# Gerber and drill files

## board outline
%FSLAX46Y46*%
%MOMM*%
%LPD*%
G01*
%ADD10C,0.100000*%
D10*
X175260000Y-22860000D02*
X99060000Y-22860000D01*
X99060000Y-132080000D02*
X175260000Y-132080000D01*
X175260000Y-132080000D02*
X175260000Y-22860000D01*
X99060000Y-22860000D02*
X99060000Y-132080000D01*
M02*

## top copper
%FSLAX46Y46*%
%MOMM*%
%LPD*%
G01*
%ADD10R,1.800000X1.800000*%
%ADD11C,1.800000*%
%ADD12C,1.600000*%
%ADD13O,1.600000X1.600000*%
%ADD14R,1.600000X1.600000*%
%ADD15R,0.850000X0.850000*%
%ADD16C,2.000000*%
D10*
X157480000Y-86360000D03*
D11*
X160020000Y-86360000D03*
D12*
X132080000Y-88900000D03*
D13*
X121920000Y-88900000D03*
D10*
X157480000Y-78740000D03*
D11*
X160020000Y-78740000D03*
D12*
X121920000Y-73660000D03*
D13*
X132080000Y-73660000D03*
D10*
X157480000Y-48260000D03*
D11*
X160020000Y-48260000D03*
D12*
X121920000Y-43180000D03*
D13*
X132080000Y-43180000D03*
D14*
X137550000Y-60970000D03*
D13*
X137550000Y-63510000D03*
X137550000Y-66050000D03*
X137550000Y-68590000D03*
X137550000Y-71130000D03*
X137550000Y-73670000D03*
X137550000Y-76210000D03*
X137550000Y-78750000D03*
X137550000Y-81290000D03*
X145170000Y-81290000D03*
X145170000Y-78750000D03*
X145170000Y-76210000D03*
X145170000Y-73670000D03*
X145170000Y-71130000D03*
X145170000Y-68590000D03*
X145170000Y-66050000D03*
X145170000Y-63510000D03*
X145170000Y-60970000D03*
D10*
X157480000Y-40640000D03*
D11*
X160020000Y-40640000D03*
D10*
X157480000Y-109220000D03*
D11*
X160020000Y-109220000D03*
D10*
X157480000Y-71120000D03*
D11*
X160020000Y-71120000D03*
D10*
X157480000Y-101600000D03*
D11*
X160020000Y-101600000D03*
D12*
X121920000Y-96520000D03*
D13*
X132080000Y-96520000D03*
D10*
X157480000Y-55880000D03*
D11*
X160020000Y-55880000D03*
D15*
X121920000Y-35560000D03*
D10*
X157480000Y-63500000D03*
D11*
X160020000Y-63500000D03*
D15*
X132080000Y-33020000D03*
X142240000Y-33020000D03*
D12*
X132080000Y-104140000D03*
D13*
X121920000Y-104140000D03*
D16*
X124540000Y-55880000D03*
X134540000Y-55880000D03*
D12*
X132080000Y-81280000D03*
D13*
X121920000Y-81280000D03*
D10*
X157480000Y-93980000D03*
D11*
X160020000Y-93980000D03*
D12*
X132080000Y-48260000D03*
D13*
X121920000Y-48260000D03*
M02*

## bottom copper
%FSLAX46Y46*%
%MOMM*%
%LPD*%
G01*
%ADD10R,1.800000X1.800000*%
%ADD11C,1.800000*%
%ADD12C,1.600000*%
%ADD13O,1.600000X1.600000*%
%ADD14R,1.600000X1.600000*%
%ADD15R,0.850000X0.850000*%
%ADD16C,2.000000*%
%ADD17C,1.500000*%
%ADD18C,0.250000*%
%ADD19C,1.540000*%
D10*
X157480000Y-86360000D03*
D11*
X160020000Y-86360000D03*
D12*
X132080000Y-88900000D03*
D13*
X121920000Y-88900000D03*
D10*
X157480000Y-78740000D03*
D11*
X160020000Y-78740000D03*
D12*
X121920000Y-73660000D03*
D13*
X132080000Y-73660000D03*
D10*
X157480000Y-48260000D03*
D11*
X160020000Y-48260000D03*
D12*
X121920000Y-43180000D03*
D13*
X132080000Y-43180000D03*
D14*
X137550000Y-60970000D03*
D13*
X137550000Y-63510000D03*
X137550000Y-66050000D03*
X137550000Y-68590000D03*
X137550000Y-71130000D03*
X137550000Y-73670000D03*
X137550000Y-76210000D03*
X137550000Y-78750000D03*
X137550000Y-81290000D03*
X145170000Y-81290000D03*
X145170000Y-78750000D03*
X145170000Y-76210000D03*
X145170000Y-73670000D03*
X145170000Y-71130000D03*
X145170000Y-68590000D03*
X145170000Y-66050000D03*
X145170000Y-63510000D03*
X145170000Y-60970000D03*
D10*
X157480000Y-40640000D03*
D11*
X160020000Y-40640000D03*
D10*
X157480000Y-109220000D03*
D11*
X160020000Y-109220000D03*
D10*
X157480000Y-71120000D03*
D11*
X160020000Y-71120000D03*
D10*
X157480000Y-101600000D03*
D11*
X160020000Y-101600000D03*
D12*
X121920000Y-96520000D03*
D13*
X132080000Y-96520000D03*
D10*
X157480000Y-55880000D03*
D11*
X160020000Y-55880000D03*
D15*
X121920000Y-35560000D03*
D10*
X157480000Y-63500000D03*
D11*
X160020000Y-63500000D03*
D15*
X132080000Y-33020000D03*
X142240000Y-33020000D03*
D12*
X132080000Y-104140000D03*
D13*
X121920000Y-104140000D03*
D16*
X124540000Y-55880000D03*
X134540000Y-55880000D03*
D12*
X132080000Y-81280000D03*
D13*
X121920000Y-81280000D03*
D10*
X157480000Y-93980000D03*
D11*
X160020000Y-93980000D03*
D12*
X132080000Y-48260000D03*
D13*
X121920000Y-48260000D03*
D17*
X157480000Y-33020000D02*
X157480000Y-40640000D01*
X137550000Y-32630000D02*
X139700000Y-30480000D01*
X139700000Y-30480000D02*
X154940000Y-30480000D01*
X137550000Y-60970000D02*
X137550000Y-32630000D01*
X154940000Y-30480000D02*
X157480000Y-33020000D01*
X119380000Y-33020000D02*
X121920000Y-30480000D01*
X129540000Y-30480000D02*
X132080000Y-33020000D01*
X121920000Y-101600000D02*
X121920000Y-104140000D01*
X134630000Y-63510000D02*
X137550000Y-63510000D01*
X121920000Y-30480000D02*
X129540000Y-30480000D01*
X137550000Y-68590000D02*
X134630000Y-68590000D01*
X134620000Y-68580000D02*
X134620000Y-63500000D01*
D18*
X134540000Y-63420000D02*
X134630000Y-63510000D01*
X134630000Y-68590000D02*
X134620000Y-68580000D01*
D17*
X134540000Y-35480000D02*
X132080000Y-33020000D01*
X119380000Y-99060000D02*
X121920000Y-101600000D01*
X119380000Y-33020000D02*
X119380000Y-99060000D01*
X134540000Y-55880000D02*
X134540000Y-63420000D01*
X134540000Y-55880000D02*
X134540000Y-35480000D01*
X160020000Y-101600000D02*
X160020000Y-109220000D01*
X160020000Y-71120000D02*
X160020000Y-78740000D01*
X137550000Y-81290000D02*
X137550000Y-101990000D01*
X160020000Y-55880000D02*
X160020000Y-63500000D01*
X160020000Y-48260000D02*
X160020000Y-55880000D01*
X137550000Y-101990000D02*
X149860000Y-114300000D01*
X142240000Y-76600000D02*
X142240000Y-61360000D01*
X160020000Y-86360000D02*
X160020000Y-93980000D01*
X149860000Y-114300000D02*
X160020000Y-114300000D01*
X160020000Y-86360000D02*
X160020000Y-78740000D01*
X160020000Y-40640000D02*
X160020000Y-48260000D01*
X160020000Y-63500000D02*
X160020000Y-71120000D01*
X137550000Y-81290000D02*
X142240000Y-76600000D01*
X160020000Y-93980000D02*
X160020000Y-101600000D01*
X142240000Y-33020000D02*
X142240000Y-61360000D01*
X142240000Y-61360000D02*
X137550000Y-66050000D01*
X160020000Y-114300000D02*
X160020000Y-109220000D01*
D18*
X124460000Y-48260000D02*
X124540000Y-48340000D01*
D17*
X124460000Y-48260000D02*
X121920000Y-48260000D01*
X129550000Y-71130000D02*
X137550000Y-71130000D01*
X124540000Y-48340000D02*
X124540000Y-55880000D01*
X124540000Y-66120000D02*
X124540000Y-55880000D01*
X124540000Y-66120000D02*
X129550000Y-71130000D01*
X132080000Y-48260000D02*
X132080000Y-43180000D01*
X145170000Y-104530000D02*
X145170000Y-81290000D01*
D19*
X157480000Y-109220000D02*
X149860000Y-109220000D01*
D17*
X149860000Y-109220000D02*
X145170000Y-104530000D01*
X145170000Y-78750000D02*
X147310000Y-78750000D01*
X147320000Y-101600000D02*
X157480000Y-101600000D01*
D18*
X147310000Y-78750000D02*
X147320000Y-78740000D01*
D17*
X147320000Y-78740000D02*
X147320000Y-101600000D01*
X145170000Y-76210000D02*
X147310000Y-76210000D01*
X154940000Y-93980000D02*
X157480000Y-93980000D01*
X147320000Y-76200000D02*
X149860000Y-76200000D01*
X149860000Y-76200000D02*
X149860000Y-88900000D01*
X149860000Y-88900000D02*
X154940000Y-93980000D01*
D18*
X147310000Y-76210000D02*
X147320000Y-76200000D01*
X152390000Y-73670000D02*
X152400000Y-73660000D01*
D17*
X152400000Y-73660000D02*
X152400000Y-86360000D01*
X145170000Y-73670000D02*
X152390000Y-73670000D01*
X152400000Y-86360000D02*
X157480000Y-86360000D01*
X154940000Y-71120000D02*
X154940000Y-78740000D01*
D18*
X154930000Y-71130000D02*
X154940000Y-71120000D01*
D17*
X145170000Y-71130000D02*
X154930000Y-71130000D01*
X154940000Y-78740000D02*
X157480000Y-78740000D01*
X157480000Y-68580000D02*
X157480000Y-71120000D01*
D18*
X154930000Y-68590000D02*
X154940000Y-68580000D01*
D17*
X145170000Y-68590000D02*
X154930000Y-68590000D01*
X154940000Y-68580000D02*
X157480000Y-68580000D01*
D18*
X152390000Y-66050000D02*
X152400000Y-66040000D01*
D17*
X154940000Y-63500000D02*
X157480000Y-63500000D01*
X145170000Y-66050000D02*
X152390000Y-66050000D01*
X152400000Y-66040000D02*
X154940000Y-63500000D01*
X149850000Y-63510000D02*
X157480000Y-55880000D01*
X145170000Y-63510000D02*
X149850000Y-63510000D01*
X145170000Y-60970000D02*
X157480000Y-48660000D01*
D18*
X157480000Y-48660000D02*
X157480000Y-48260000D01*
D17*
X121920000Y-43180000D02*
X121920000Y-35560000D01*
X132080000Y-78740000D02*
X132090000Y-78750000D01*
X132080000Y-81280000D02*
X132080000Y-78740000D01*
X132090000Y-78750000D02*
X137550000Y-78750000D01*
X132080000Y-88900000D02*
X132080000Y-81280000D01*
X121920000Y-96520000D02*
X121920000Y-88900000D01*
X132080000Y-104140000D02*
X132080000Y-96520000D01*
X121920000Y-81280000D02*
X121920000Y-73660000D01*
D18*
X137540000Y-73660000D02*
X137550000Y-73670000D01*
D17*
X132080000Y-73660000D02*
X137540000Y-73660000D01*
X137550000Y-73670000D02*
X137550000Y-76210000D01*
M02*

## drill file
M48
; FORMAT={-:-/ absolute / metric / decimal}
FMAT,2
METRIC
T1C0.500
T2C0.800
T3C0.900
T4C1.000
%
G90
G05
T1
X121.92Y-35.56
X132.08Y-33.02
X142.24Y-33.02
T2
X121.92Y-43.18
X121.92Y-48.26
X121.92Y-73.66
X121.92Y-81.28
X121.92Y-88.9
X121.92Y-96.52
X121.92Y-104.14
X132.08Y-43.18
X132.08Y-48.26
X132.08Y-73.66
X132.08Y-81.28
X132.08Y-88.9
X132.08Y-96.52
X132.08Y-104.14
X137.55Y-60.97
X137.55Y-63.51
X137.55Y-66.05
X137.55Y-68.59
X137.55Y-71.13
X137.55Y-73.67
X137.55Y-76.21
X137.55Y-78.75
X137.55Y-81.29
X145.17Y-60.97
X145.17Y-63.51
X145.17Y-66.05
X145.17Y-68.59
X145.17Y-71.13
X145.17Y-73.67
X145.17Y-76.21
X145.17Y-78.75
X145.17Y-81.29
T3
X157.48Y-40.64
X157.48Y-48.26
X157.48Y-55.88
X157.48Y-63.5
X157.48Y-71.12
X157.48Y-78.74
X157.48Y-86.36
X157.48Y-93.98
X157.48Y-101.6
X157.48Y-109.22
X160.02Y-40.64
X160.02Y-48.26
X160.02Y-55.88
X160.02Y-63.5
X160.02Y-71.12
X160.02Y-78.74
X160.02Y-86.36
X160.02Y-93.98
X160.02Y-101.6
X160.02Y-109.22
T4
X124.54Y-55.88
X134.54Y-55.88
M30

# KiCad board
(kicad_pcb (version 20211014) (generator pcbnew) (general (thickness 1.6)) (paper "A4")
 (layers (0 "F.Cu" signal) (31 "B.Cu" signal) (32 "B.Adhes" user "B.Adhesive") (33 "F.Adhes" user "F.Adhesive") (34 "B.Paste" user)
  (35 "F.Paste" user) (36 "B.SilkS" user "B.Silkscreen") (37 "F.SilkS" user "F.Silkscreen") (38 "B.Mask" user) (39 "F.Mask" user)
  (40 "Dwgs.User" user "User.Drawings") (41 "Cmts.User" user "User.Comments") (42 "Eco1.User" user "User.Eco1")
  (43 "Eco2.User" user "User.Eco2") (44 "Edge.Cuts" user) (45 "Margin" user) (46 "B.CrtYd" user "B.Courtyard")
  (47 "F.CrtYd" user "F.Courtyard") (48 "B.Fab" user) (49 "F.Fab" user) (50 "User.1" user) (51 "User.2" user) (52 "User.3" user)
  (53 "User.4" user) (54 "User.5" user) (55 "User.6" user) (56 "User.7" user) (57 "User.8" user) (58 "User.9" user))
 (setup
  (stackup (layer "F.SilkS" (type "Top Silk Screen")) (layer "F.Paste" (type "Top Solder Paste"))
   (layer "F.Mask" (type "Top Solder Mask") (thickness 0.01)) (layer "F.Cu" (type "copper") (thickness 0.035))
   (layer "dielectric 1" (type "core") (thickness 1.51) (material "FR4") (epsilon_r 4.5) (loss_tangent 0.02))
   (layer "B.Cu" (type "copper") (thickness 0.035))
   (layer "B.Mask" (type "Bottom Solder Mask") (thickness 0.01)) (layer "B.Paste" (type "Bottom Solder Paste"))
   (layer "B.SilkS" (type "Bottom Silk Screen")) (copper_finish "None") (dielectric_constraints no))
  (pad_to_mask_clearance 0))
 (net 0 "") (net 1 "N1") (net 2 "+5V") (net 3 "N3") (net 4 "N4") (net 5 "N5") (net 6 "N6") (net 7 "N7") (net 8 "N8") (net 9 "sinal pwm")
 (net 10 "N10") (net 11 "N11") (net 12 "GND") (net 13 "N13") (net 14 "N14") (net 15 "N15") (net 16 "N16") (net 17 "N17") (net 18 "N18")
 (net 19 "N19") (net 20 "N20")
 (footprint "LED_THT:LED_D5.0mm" (layer "F.Cu") (at 157.48 86.36)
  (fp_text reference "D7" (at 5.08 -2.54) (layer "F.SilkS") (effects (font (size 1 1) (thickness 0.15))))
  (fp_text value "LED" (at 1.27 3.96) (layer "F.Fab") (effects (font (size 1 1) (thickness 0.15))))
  (pad "1" thru_hole rect (at 0 0) (size 1.8 1.8) (drill 0.9) (layers *.Cu *.Mask) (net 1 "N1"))
  (pad "2" thru_hole circle (at 2.54 0) (size 1.8 1.8) (drill 0.9) (layers *.Cu *.Mask) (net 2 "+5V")))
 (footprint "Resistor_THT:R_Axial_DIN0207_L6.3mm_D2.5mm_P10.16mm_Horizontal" (layer "F.Cu") (at 132.08 88.9 180)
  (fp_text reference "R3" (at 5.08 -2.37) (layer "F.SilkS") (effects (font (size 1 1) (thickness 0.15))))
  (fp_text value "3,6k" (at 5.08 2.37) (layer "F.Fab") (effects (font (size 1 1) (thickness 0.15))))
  (pad "1" thru_hole circle (at 0 0 180) (size 1.6 1.6) (drill 0.8) (layers *.Cu *.Mask) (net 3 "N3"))
  (pad "2" thru_hole oval (at 10.16 0 180) (size 1.6 1.6) (drill 0.8) (layers *.Cu *.Mask) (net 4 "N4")))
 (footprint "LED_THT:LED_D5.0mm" (layer "F.Cu") (at 157.48 78.74)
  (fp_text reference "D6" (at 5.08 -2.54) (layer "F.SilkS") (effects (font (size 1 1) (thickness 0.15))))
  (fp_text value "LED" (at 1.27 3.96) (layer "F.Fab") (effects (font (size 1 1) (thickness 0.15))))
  (pad "1" thru_hole rect (at 0 0) (size 1.8 1.8) (drill 0.9) (layers *.Cu *.Mask) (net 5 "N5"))
  (pad "2" thru_hole circle (at 2.54 0) (size 1.8 1.8) (drill 0.9) (layers *.Cu *.Mask) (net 2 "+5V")))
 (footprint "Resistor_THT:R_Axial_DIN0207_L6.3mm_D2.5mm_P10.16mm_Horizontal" (layer "F.Cu") (at 121.92 73.66)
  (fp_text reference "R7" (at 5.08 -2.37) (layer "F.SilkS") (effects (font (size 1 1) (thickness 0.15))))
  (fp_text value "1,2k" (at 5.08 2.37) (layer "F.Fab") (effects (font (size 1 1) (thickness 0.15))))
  (pad "1" thru_hole circle (at 0 0) (size 1.6 1.6) (drill 0.8) (layers *.Cu *.Mask) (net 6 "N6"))
  (pad "2" thru_hole oval (at 10.16 0) (size 1.6 1.6) (drill 0.8) (layers *.Cu *.Mask) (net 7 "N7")))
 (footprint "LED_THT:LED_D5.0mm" (layer "F.Cu") (at 157.48 48.26)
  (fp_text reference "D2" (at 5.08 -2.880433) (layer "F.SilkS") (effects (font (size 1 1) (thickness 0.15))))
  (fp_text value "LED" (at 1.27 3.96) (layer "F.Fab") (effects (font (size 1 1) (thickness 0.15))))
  (pad "1" thru_hole rect (at 0 0) (size 1.8 1.8) (drill 0.9) (layers *.Cu *.Mask) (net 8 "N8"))
  (pad "2" thru_hole circle (at 2.54 0) (size 1.8 1.8) (drill 0.9) (layers *.Cu *.Mask) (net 2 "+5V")))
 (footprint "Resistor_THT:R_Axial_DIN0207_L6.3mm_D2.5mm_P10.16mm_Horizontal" (layer "F.Cu") (at 121.92 43.18)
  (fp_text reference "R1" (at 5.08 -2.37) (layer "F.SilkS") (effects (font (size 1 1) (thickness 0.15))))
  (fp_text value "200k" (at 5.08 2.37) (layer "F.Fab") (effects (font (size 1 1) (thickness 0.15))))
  (pad "1" thru_hole circle (at 0 0) (size 1.6 1.6) (drill 0.8) (layers *.Cu *.Mask) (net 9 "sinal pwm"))
  (pad "2" thru_hole oval (at 10.16 0) (size 1.6 1.6) (drill 0.8) (layers *.Cu *.Mask) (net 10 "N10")))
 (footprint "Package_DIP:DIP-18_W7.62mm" (layer "F.Cu") (at 137.55 60.97)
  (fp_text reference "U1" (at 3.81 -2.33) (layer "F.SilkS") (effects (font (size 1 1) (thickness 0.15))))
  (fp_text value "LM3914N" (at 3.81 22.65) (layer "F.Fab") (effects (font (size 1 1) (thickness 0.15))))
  (pad "1" thru_hole rect (at 0 0) (size 1.6 1.6) (drill 0.8) (layers *.Cu *.Mask) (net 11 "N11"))
  (pad "2" thru_hole oval (at 0 2.54) (size 1.6 1.6) (drill 0.8) (layers *.Cu *.Mask) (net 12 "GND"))
  (pad "3" thru_hole oval (at 0 5.08) (size 1.6 1.6) (drill 0.8) (layers *.Cu *.Mask) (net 2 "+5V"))
  (pad "4" thru_hole oval (at 0 7.62) (size 1.6 1.6) (drill 0.8) (layers *.Cu *.Mask) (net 12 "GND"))
  (pad "5" thru_hole oval (at 0 10.16) (size 1.6 1.6) (drill 0.8) (layers *.Cu *.Mask) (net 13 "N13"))
  (pad "6" thru_hole oval (at 0 12.7) (size 1.6 1.6) (drill 0.8) (layers *.Cu *.Mask) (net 7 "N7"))
  (pad "7" thru_hole oval (at 0 15.24) (size 1.6 1.6) (drill 0.8) (layers *.Cu *.Mask) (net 7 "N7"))
  (pad "8" thru_hole oval (at 0 17.78) (size 1.6 1.6) (drill 0.8) (layers *.Cu *.Mask) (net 3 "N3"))
  (pad "9" thru_hole oval (at 0 20.32) (size 1.6 1.6) (drill 0.8) (layers *.Cu *.Mask) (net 2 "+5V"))
  (pad "10" thru_hole oval (at 7.62 20.32) (size 1.6 1.6) (drill 0.8) (layers *.Cu *.Mask) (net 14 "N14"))
  (pad "11" thru_hole oval (at 7.62 17.78) (size 1.6 1.6) (drill 0.8) (layers *.Cu *.Mask) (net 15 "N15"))
  (pad "12" thru_hole oval (at 7.62 15.24) (size 1.6 1.6) (drill 0.8) (layers *.Cu *.Mask) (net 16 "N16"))
  (pad "13" thru_hole oval (at 7.62 12.7) (size 1.6 1.6) (drill 0.8) (layers *.Cu *.Mask) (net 1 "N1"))
  (pad "14" thru_hole oval (at 7.62 10.16) (size 1.6 1.6) (drill 0.8) (layers *.Cu *.Mask) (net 5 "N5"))
  (pad "15" thru_hole oval (at 7.62 7.62) (size 1.6 1.6) (drill 0.8) (layers *.Cu *.Mask) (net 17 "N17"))
  (pad "16" thru_hole oval (at 7.62 5.08) (size 1.6 1.6) (drill 0.8) (layers *.Cu *.Mask) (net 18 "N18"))
  (pad "17" thru_hole oval (at 7.62 2.54) (size 1.6 1.6) (drill 0.8) (layers *.Cu *.Mask) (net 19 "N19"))
  (pad "18" thru_hole oval (at 7.62 0) (size 1.6 1.6) (drill 0.8) (layers *.Cu *.Mask) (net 8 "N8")))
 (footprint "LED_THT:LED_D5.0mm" (layer "F.Cu") (at 157.48 40.64)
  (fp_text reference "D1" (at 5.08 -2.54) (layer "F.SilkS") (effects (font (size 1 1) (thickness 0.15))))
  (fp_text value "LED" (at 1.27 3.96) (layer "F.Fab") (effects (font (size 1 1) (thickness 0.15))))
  (pad "1" thru_hole rect (at 0 0) (size 1.8 1.8) (drill 0.9) (layers *.Cu *.Mask) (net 11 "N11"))
  (pad "2" thru_hole circle (at 2.54 0) (size 1.8 1.8) (drill 0.9) (layers *.Cu *.Mask) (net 2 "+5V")))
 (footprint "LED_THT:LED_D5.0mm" (layer "F.Cu") (at 157.48 109.22)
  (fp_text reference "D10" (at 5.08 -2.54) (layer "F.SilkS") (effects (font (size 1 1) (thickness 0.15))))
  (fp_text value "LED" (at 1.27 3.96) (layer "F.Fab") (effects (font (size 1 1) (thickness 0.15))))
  (pad "1" thru_hole rect (at 0 0) (size 1.8 1.8) (drill 0.9) (layers *.Cu *.Mask) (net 14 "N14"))
  (pad "2" thru_hole circle (at 2.54 0) (size 1.8 1.8) (drill 0.9) (layers *.Cu *.Mask) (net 2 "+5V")))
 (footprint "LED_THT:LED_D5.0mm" (layer "F.Cu") (at 157.48 71.12)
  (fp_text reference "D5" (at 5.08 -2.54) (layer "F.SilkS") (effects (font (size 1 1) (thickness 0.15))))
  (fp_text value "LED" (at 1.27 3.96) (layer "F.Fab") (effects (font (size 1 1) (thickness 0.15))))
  (pad "1" thru_hole rect (at 0 0) (size 1.8 1.8) (drill 0.9) (layers *.Cu *.Mask) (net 17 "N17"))
  (pad "2" thru_hole circle (at 2.54 0) (size 1.8 1.8) (drill 0.9) (layers *.Cu *.Mask) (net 2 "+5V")))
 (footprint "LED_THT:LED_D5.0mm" (layer "F.Cu") (at 157.48 101.6)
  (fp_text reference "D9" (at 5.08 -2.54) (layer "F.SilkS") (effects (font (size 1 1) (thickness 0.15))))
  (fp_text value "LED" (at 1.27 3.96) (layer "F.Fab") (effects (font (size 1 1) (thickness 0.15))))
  (pad "1" thru_hole rect (at 0 0) (size 1.8 1.8) (drill 0.9) (layers *.Cu *.Mask) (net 15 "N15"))
  (pad "2" thru_hole circle (at 2.54 0) (size 1.8 1.8) (drill 0.9) (layers *.Cu *.Mask) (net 2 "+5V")))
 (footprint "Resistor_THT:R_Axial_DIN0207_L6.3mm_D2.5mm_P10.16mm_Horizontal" (layer "F.Cu") (at 121.92 96.52)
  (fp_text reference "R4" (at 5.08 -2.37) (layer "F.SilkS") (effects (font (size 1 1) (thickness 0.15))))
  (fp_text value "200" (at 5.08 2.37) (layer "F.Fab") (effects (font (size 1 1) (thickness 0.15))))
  (pad "1" thru_hole circle (at 0 0) (size 1.6 1.6) (drill 0.8) (layers *.Cu *.Mask) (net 4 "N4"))
  (pad "2" thru_hole oval (at 10.16 0) (size 1.6 1.6) (drill 0.8) (layers *.Cu *.Mask) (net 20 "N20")))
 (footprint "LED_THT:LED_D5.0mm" (layer "F.Cu") (at 157.48 55.88)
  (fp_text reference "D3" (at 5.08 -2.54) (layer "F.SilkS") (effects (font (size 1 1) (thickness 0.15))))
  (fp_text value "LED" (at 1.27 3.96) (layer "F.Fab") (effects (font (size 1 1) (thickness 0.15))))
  (pad "1" thru_hole rect (at 0 0) (size 1.8 1.8) (drill 0.9) (layers *.Cu *.Mask) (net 19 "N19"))
  (pad "2" thru_hole circle (at 2.54 0) (size 1.8 1.8) (drill 0.9) (layers *.Cu *.Mask) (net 2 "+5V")))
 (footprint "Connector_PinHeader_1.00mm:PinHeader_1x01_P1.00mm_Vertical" (layer "F.Cu") (at 121.92 35.56)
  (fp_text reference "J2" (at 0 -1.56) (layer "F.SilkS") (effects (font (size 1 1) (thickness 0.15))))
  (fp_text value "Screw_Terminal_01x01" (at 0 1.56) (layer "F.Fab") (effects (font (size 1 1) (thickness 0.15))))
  (pad "1" thru_hole rect (at 0 0) (size 0.85 0.85) (drill 0.5) (layers *.Cu *.Mask) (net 9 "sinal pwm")))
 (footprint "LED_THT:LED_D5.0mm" (layer "F.Cu") (at 157.48 63.5)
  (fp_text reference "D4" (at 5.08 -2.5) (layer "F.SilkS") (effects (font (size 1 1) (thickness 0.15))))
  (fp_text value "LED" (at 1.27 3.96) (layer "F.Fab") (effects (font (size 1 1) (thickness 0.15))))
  (pad "1" thru_hole rect (at 0 0) (size 1.8 1.8) (drill 0.9) (layers *.Cu *.Mask) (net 18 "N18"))
  (pad "2" thru_hole circle (at 2.54 0) (size 1.8 1.8) (drill 0.9) (layers *.Cu *.Mask) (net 2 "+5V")))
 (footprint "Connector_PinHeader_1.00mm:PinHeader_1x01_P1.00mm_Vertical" (layer "F.Cu") (at 132.08 33.02)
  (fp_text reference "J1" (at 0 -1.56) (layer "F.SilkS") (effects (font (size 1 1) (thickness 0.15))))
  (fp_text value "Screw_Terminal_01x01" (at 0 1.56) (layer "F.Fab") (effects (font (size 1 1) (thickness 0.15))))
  (pad "1" thru_hole rect (at 0 0) (size 0.85 0.85) (drill 0.5) (layers *.Cu *.Mask) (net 12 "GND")))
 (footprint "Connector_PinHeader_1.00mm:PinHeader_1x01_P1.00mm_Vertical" (layer "F.Cu") (at 142.24 33.02)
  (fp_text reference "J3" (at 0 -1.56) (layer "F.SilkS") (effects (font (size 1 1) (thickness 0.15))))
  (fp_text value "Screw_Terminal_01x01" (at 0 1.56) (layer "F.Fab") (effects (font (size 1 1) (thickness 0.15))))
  (pad "1" thru_hole rect (at 0 0) (size 0.85 0.85) (drill 0.5) (layers *.Cu *.Mask) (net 2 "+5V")))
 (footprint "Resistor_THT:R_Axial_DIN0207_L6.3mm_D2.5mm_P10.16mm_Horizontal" (layer "F.Cu") (at 132.08 104.14 180)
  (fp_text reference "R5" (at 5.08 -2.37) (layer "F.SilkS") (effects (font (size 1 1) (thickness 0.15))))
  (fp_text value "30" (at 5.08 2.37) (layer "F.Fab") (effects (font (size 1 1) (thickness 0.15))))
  (pad "1" thru_hole circle (at 0 0 180) (size 1.6 1.6) (drill 0.8) (layers *.Cu *.Mask) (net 20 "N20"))
  (pad "2" thru_hole oval (at 10.16 0 180) (size 1.6 1.6) (drill 0.8) (layers *.Cu *.Mask) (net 12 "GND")))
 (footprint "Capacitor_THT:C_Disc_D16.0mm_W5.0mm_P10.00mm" (layer "F.Cu") (at 124.54 55.88)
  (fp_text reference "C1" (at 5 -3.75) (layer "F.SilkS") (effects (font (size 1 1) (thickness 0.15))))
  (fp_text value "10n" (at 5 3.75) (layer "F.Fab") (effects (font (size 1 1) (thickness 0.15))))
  (pad "1" thru_hole circle (at 0 0) (size 2 2) (drill 1) (layers *.Cu *.Mask) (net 13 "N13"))
  (pad "2" thru_hole circle (at 10 0) (size 2 2) (drill 1) (layers *.Cu *.Mask) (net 12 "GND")))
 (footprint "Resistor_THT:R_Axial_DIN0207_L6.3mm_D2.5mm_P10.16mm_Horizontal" (layer "F.Cu") (at 132.08 81.28 180)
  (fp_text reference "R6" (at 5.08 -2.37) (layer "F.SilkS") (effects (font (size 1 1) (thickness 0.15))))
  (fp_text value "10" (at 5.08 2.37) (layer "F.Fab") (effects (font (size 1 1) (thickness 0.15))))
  (pad "1" thru_hole circle (at 0 0 180) (size 1.6 1.6) (drill 0.8) (layers *.Cu *.Mask) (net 3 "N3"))
  (pad "2" thru_hole oval (at 10.16 0 180) (size 1.6 1.6) (drill 0.8) (layers *.Cu *.Mask) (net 6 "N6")))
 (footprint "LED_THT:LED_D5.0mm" (layer "F.Cu") (at 157.48 93.98)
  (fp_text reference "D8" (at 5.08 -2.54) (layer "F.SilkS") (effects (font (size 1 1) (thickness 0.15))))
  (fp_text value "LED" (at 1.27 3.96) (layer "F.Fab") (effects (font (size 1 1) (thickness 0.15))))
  (pad "1" thru_hole rect (at 0 0) (size 1.8 1.8) (drill 0.9) (layers *.Cu *.Mask) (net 16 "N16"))
  (pad "2" thru_hole circle (at 2.54 0) (size 1.8 1.8) (drill 0.9) (layers *.Cu *.Mask) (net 2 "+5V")))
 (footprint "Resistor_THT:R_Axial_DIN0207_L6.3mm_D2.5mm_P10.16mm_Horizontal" (layer "F.Cu") (at 132.08 48.26 180)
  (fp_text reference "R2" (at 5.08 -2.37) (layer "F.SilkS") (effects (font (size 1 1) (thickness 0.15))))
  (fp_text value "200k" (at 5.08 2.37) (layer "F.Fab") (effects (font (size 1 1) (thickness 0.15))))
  (pad "1" thru_hole circle (at 0 0 180) (size 1.6 1.6) (drill 0.8) (layers *.Cu *.Mask) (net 10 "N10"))
  (pad "2" thru_hole oval (at 10.16 0 180) (size 1.6 1.6) (drill 0.8) (layers *.Cu *.Mask) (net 13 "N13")))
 (gr_rect (start 177.8 134.62) (end 177.8 134.62) (layer "B.Cu") (width 0.2) (fill none))
 (gr_line (start 175.26 22.86) (end 99.06 22.86) (layer "Edge.Cuts") (width 0.1))
 (gr_line (start 99.06 132.08) (end 175.26 132.08) (layer "Edge.Cuts") (width 0.1))
 (gr_line (start 175.26 132.08) (end 175.26 22.86) (layer "Edge.Cuts") (width 0.1))
 (gr_line (start 99.06 22.86) (end 99.06 132.08) (layer "Edge.Cuts") (width 0.1))
 (segment (start 157.48 33.02) (end 157.48 40.64) (width 1.5) (layer "B.Cu") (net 11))
 (segment (start 137.55 32.63) (end 139.7 30.48) (width 1.5) (layer "B.Cu") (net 11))
 (segment (start 139.7 30.48) (end 154.94 30.48) (width 1.5) (layer "B.Cu") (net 11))
 (segment (start 137.55 60.97) (end 137.55 32.63) (width 1.5) (layer "B.Cu") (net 11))
 (segment (start 154.94 30.48) (end 157.48 33.02) (width 1.5) (layer "B.Cu") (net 11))
 (segment (start 119.38 33.02) (end 121.92 30.48) (width 1.5) (layer "B.Cu") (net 12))
 (segment (start 129.54 30.48) (end 132.08 33.02) (width 1.5) (layer "B.Cu") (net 12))
 (segment (start 121.92 101.6) (end 121.92 104.14) (width 1.5) (layer "B.Cu") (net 12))
 (segment (start 134.63 63.51) (end 137.55 63.51) (width 1.5) (layer "B.Cu") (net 12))
 (segment (start 121.92 30.48) (end 129.54 30.48) (width 1.5) (layer "B.Cu") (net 12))
 (segment (start 137.55 68.59) (end 134.63 68.59) (width 1.5) (layer "B.Cu") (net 12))
 (segment (start 134.62 68.58) (end 134.62 63.5) (width 1.5) (layer "B.Cu") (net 12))
 (segment (start 134.54 63.42) (end 134.63 63.51) (width 0.25) (layer "B.Cu") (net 12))
 (segment (start 134.63 68.59) (end 134.62 68.58) (width 0.25) (layer "B.Cu") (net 12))
 (segment (start 134.54 35.48) (end 132.08 33.02) (width 1.5) (layer "B.Cu") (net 12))
 (segment (start 119.38 99.06) (end 121.92 101.6) (width 1.5) (layer "B.Cu") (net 12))
 (segment (start 119.38 33.02) (end 119.38 99.06) (width 1.5) (layer "B.Cu") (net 12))
 (segment (start 134.54 55.88) (end 134.54 63.42) (width 1.5) (layer "B.Cu") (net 12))
 (segment (start 134.54 55.88) (end 134.54 35.48) (width 1.5) (layer "B.Cu") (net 12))
 (segment (start 160.02 101.6) (end 160.02 109.22) (width 1.5) (layer "B.Cu") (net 2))
 (segment (start 160.02 71.12) (end 160.02 78.74) (width 1.5) (layer "B.Cu") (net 2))
 (segment (start 137.55 81.29) (end 137.55 101.99) (width 1.5) (layer "B.Cu") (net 2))
 (segment (start 160.02 55.88) (end 160.02 63.5) (width 1.5) (layer "B.Cu") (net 2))
 (segment (start 160.02 48.26) (end 160.02 55.88) (width 1.5) (layer "B.Cu") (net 2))
 (segment (start 137.55 101.99) (end 149.86 114.3) (width 1.5) (layer "B.Cu") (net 2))
 (segment (start 142.24 76.6) (end 142.24 61.36) (width 1.5) (layer "B.Cu") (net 2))
 (segment (start 160.02 86.36) (end 160.02 93.98) (width 1.5) (layer "B.Cu") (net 2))
 (segment (start 149.86 114.3) (end 160.02 114.3) (width 1.5) (layer "B.Cu") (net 2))
 (segment (start 160.02 86.36) (end 160.02 78.74) (width 1.5) (layer "B.Cu") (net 2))
 (segment (start 160.02 40.64) (end 160.02 48.26) (width 1.5) (layer "B.Cu") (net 2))
 (segment (start 160.02 63.5) (end 160.02 71.12) (width 1.5) (layer "B.Cu") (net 2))
 (segment (start 137.55 81.29) (end 142.24 76.6) (width 1.5) (layer "B.Cu") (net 2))
 (segment (start 160.02 93.98) (end 160.02 101.6) (width 1.5) (layer "B.Cu") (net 2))
 (segment (start 142.24 33.02) (end 142.24 61.36) (width 1.5) (layer "B.Cu") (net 2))
 (segment (start 142.24 61.36) (end 137.55 66.05) (width 1.5) (layer "B.Cu") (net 2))
 (segment (start 160.02 114.3) (end 160.02 109.22) (width 1.5) (layer "B.Cu") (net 2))
 (segment (start 124.46 48.26) (end 124.54 48.34) (width 0.25) (layer "B.Cu") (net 13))
 (segment (start 124.46 48.26) (end 121.92 48.26) (width 1.5) (layer "B.Cu") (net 13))
 (segment (start 129.55 71.13) (end 137.55 71.13) (width 1.5) (layer "B.Cu") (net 13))
 (segment (start 124.54 48.34) (end 124.54 55.88) (width 1.5) (layer "B.Cu") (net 13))
 (segment (start 124.54 66.12) (end 124.54 55.88) (width 1.5) (layer "B.Cu") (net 13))
 (segment (start 124.54 66.12) (end 129.55 71.13) (width 1.5) (layer "B.Cu") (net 13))
 (segment (start 132.08 48.26) (end 132.08 43.18) (width 1.5) (layer "B.Cu") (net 10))
 (segment (start 145.17 104.53) (end 145.17 81.29) (width 1.5) (layer "B.Cu") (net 14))
 (segment (start 157.48 109.22) (end 149.86 109.22) (width 1.54) (layer "B.Cu") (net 14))
 (segment (start 149.86 109.22) (end 145.17 104.53) (width 1.5) (layer "B.Cu") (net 14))
 (segment (start 145.17 78.75) (end 147.31 78.75) (width 1.5) (layer "B.Cu") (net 15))
 (segment (start 147.32 101.6) (end 157.48 101.6) (width 1.5) (layer "B.Cu") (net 15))
 (segment (start 147.31 78.75) (end 147.32 78.74) (width 0.25) (layer "B.Cu") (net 15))
 (segment (start 147.32 78.74) (end 147.32 101.6) (width 1.5) (layer "B.Cu") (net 15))
 (segment (start 145.17 76.21) (end 147.31 76.21) (width 1.5) (layer "B.Cu") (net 16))
 (segment (start 154.94 93.98) (end 157.48 93.98) (width 1.5) (layer "B.Cu") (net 16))
 (segment (start 147.32 76.2) (end 149.86 76.2) (width 1.5) (layer "B.Cu") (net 16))
 (segment (start 149.86 76.2) (end 149.86 88.9) (width 1.5) (layer "B.Cu") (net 16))
 (segment (start 149.86 88.9) (end 154.94 93.98) (width 1.5) (layer "B.Cu") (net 16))
 (segment (start 147.31 76.21) (end 147.32 76.2) (width 0.25) (layer "B.Cu") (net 16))
 (segment (start 152.39 73.67) (end 152.4 73.66) (width 0.25) (layer "B.Cu") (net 1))
 (segment (start 152.4 73.66) (end 152.4 86.36) (width 1.5) (layer "B.Cu") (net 1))
 (segment (start 145.17 73.67) (end 152.39 73.67) (width 1.5) (layer "B.Cu") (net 1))
 (segment (start 152.4 86.36) (end 157.48 86.36) (width 1.5) (layer "B.Cu") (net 1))
 (segment (start 154.94 71.12) (end 154.94 78.74) (width 1.5) (layer "B.Cu") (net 5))
 (segment (start 154.93 71.13) (end 154.94 71.12) (width 0.25) (layer "B.Cu") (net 5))
 (segment (start 145.17 71.13) (end 154.93 71.13) (width 1.5) (layer "B.Cu") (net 5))
 (segment (start 154.94 78.74) (end 157.48 78.74) (width 1.5) (layer "B.Cu") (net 5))
 (segment (start 157.48 68.58) (end 157.48 71.12) (width 1.5) (layer "B.Cu") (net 17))
 (segment (start 154.93 68.59) (end 154.94 68.58) (width 0.25) (layer "B.Cu") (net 17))
 (segment (start 145.17 68.59) (end 154.93 68.59) (width 1.5) (layer "B.Cu") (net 17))
 (segment (start 154.94 68.58) (end 157.48 68.58) (width 1.5) (layer "B.Cu") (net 17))
 (segment (start 152.39 66.05) (end 152.4 66.04) (width 0.25) (layer "B.Cu") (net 18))
 (segment (start 154.94 63.5) (end 157.48 63.5) (width 1.5) (layer "B.Cu") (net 18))
 (segment (start 145.17 66.05) (end 152.39 66.05) (width 1.5) (layer "B.Cu") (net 18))
 (segment (start 152.4 66.04) (end 154.94 63.5) (width 1.5) (layer "B.Cu") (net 18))
 (segment (start 149.85 63.51) (end 157.48 55.88) (width 1.5) (layer "B.Cu") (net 19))
 (segment (start 145.17 63.51) (end 149.85 63.51) (width 1.5) (layer "B.Cu") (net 19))
 (segment (start 145.17 60.97) (end 157.48 48.66) (width 1.5) (layer "B.Cu") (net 8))
 (segment (start 157.48 48.66) (end 157.48 48.26) (width 0.25) (layer "B.Cu") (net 8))
 (segment (start 121.92 43.18) (end 121.92 35.56) (width 1.5) (layer "B.Cu") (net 9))
 (segment (start 132.08 78.74) (end 132.09 78.75) (width 1.5) (layer "B.Cu") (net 3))
 (segment (start 132.08 81.28) (end 132.08 78.74) (width 1.5) (layer "B.Cu") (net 3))
 (segment (start 132.09 78.75) (end 137.55 78.75) (width 1.5) (layer "B.Cu") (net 3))
 (segment (start 132.08 88.9) (end 132.08 81.28) (width 1.5) (layer "B.Cu") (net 3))
 (segment (start 121.92 96.52) (end 121.92 88.9) (width 1.5) (layer "B.Cu") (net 4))
 (segment (start 132.08 104.14) (end 132.08 96.52) (width 1.5) (layer "B.Cu") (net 20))
 (segment (start 121.92 81.28) (end 121.92 73.66) (width 1.5) (layer "B.Cu") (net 6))
 (segment (start 137.54 73.66) (end 137.55 73.67) (width 0.25) (layer "B.Cu") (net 7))
 (segment (start 132.08 73.66) (end 137.54 73.66) (width 1.5) (layer "B.Cu") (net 7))
 (segment (start 137.55 73.67) (end 137.55 76.21) (width 1.5) (layer "B.Cu") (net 7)))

